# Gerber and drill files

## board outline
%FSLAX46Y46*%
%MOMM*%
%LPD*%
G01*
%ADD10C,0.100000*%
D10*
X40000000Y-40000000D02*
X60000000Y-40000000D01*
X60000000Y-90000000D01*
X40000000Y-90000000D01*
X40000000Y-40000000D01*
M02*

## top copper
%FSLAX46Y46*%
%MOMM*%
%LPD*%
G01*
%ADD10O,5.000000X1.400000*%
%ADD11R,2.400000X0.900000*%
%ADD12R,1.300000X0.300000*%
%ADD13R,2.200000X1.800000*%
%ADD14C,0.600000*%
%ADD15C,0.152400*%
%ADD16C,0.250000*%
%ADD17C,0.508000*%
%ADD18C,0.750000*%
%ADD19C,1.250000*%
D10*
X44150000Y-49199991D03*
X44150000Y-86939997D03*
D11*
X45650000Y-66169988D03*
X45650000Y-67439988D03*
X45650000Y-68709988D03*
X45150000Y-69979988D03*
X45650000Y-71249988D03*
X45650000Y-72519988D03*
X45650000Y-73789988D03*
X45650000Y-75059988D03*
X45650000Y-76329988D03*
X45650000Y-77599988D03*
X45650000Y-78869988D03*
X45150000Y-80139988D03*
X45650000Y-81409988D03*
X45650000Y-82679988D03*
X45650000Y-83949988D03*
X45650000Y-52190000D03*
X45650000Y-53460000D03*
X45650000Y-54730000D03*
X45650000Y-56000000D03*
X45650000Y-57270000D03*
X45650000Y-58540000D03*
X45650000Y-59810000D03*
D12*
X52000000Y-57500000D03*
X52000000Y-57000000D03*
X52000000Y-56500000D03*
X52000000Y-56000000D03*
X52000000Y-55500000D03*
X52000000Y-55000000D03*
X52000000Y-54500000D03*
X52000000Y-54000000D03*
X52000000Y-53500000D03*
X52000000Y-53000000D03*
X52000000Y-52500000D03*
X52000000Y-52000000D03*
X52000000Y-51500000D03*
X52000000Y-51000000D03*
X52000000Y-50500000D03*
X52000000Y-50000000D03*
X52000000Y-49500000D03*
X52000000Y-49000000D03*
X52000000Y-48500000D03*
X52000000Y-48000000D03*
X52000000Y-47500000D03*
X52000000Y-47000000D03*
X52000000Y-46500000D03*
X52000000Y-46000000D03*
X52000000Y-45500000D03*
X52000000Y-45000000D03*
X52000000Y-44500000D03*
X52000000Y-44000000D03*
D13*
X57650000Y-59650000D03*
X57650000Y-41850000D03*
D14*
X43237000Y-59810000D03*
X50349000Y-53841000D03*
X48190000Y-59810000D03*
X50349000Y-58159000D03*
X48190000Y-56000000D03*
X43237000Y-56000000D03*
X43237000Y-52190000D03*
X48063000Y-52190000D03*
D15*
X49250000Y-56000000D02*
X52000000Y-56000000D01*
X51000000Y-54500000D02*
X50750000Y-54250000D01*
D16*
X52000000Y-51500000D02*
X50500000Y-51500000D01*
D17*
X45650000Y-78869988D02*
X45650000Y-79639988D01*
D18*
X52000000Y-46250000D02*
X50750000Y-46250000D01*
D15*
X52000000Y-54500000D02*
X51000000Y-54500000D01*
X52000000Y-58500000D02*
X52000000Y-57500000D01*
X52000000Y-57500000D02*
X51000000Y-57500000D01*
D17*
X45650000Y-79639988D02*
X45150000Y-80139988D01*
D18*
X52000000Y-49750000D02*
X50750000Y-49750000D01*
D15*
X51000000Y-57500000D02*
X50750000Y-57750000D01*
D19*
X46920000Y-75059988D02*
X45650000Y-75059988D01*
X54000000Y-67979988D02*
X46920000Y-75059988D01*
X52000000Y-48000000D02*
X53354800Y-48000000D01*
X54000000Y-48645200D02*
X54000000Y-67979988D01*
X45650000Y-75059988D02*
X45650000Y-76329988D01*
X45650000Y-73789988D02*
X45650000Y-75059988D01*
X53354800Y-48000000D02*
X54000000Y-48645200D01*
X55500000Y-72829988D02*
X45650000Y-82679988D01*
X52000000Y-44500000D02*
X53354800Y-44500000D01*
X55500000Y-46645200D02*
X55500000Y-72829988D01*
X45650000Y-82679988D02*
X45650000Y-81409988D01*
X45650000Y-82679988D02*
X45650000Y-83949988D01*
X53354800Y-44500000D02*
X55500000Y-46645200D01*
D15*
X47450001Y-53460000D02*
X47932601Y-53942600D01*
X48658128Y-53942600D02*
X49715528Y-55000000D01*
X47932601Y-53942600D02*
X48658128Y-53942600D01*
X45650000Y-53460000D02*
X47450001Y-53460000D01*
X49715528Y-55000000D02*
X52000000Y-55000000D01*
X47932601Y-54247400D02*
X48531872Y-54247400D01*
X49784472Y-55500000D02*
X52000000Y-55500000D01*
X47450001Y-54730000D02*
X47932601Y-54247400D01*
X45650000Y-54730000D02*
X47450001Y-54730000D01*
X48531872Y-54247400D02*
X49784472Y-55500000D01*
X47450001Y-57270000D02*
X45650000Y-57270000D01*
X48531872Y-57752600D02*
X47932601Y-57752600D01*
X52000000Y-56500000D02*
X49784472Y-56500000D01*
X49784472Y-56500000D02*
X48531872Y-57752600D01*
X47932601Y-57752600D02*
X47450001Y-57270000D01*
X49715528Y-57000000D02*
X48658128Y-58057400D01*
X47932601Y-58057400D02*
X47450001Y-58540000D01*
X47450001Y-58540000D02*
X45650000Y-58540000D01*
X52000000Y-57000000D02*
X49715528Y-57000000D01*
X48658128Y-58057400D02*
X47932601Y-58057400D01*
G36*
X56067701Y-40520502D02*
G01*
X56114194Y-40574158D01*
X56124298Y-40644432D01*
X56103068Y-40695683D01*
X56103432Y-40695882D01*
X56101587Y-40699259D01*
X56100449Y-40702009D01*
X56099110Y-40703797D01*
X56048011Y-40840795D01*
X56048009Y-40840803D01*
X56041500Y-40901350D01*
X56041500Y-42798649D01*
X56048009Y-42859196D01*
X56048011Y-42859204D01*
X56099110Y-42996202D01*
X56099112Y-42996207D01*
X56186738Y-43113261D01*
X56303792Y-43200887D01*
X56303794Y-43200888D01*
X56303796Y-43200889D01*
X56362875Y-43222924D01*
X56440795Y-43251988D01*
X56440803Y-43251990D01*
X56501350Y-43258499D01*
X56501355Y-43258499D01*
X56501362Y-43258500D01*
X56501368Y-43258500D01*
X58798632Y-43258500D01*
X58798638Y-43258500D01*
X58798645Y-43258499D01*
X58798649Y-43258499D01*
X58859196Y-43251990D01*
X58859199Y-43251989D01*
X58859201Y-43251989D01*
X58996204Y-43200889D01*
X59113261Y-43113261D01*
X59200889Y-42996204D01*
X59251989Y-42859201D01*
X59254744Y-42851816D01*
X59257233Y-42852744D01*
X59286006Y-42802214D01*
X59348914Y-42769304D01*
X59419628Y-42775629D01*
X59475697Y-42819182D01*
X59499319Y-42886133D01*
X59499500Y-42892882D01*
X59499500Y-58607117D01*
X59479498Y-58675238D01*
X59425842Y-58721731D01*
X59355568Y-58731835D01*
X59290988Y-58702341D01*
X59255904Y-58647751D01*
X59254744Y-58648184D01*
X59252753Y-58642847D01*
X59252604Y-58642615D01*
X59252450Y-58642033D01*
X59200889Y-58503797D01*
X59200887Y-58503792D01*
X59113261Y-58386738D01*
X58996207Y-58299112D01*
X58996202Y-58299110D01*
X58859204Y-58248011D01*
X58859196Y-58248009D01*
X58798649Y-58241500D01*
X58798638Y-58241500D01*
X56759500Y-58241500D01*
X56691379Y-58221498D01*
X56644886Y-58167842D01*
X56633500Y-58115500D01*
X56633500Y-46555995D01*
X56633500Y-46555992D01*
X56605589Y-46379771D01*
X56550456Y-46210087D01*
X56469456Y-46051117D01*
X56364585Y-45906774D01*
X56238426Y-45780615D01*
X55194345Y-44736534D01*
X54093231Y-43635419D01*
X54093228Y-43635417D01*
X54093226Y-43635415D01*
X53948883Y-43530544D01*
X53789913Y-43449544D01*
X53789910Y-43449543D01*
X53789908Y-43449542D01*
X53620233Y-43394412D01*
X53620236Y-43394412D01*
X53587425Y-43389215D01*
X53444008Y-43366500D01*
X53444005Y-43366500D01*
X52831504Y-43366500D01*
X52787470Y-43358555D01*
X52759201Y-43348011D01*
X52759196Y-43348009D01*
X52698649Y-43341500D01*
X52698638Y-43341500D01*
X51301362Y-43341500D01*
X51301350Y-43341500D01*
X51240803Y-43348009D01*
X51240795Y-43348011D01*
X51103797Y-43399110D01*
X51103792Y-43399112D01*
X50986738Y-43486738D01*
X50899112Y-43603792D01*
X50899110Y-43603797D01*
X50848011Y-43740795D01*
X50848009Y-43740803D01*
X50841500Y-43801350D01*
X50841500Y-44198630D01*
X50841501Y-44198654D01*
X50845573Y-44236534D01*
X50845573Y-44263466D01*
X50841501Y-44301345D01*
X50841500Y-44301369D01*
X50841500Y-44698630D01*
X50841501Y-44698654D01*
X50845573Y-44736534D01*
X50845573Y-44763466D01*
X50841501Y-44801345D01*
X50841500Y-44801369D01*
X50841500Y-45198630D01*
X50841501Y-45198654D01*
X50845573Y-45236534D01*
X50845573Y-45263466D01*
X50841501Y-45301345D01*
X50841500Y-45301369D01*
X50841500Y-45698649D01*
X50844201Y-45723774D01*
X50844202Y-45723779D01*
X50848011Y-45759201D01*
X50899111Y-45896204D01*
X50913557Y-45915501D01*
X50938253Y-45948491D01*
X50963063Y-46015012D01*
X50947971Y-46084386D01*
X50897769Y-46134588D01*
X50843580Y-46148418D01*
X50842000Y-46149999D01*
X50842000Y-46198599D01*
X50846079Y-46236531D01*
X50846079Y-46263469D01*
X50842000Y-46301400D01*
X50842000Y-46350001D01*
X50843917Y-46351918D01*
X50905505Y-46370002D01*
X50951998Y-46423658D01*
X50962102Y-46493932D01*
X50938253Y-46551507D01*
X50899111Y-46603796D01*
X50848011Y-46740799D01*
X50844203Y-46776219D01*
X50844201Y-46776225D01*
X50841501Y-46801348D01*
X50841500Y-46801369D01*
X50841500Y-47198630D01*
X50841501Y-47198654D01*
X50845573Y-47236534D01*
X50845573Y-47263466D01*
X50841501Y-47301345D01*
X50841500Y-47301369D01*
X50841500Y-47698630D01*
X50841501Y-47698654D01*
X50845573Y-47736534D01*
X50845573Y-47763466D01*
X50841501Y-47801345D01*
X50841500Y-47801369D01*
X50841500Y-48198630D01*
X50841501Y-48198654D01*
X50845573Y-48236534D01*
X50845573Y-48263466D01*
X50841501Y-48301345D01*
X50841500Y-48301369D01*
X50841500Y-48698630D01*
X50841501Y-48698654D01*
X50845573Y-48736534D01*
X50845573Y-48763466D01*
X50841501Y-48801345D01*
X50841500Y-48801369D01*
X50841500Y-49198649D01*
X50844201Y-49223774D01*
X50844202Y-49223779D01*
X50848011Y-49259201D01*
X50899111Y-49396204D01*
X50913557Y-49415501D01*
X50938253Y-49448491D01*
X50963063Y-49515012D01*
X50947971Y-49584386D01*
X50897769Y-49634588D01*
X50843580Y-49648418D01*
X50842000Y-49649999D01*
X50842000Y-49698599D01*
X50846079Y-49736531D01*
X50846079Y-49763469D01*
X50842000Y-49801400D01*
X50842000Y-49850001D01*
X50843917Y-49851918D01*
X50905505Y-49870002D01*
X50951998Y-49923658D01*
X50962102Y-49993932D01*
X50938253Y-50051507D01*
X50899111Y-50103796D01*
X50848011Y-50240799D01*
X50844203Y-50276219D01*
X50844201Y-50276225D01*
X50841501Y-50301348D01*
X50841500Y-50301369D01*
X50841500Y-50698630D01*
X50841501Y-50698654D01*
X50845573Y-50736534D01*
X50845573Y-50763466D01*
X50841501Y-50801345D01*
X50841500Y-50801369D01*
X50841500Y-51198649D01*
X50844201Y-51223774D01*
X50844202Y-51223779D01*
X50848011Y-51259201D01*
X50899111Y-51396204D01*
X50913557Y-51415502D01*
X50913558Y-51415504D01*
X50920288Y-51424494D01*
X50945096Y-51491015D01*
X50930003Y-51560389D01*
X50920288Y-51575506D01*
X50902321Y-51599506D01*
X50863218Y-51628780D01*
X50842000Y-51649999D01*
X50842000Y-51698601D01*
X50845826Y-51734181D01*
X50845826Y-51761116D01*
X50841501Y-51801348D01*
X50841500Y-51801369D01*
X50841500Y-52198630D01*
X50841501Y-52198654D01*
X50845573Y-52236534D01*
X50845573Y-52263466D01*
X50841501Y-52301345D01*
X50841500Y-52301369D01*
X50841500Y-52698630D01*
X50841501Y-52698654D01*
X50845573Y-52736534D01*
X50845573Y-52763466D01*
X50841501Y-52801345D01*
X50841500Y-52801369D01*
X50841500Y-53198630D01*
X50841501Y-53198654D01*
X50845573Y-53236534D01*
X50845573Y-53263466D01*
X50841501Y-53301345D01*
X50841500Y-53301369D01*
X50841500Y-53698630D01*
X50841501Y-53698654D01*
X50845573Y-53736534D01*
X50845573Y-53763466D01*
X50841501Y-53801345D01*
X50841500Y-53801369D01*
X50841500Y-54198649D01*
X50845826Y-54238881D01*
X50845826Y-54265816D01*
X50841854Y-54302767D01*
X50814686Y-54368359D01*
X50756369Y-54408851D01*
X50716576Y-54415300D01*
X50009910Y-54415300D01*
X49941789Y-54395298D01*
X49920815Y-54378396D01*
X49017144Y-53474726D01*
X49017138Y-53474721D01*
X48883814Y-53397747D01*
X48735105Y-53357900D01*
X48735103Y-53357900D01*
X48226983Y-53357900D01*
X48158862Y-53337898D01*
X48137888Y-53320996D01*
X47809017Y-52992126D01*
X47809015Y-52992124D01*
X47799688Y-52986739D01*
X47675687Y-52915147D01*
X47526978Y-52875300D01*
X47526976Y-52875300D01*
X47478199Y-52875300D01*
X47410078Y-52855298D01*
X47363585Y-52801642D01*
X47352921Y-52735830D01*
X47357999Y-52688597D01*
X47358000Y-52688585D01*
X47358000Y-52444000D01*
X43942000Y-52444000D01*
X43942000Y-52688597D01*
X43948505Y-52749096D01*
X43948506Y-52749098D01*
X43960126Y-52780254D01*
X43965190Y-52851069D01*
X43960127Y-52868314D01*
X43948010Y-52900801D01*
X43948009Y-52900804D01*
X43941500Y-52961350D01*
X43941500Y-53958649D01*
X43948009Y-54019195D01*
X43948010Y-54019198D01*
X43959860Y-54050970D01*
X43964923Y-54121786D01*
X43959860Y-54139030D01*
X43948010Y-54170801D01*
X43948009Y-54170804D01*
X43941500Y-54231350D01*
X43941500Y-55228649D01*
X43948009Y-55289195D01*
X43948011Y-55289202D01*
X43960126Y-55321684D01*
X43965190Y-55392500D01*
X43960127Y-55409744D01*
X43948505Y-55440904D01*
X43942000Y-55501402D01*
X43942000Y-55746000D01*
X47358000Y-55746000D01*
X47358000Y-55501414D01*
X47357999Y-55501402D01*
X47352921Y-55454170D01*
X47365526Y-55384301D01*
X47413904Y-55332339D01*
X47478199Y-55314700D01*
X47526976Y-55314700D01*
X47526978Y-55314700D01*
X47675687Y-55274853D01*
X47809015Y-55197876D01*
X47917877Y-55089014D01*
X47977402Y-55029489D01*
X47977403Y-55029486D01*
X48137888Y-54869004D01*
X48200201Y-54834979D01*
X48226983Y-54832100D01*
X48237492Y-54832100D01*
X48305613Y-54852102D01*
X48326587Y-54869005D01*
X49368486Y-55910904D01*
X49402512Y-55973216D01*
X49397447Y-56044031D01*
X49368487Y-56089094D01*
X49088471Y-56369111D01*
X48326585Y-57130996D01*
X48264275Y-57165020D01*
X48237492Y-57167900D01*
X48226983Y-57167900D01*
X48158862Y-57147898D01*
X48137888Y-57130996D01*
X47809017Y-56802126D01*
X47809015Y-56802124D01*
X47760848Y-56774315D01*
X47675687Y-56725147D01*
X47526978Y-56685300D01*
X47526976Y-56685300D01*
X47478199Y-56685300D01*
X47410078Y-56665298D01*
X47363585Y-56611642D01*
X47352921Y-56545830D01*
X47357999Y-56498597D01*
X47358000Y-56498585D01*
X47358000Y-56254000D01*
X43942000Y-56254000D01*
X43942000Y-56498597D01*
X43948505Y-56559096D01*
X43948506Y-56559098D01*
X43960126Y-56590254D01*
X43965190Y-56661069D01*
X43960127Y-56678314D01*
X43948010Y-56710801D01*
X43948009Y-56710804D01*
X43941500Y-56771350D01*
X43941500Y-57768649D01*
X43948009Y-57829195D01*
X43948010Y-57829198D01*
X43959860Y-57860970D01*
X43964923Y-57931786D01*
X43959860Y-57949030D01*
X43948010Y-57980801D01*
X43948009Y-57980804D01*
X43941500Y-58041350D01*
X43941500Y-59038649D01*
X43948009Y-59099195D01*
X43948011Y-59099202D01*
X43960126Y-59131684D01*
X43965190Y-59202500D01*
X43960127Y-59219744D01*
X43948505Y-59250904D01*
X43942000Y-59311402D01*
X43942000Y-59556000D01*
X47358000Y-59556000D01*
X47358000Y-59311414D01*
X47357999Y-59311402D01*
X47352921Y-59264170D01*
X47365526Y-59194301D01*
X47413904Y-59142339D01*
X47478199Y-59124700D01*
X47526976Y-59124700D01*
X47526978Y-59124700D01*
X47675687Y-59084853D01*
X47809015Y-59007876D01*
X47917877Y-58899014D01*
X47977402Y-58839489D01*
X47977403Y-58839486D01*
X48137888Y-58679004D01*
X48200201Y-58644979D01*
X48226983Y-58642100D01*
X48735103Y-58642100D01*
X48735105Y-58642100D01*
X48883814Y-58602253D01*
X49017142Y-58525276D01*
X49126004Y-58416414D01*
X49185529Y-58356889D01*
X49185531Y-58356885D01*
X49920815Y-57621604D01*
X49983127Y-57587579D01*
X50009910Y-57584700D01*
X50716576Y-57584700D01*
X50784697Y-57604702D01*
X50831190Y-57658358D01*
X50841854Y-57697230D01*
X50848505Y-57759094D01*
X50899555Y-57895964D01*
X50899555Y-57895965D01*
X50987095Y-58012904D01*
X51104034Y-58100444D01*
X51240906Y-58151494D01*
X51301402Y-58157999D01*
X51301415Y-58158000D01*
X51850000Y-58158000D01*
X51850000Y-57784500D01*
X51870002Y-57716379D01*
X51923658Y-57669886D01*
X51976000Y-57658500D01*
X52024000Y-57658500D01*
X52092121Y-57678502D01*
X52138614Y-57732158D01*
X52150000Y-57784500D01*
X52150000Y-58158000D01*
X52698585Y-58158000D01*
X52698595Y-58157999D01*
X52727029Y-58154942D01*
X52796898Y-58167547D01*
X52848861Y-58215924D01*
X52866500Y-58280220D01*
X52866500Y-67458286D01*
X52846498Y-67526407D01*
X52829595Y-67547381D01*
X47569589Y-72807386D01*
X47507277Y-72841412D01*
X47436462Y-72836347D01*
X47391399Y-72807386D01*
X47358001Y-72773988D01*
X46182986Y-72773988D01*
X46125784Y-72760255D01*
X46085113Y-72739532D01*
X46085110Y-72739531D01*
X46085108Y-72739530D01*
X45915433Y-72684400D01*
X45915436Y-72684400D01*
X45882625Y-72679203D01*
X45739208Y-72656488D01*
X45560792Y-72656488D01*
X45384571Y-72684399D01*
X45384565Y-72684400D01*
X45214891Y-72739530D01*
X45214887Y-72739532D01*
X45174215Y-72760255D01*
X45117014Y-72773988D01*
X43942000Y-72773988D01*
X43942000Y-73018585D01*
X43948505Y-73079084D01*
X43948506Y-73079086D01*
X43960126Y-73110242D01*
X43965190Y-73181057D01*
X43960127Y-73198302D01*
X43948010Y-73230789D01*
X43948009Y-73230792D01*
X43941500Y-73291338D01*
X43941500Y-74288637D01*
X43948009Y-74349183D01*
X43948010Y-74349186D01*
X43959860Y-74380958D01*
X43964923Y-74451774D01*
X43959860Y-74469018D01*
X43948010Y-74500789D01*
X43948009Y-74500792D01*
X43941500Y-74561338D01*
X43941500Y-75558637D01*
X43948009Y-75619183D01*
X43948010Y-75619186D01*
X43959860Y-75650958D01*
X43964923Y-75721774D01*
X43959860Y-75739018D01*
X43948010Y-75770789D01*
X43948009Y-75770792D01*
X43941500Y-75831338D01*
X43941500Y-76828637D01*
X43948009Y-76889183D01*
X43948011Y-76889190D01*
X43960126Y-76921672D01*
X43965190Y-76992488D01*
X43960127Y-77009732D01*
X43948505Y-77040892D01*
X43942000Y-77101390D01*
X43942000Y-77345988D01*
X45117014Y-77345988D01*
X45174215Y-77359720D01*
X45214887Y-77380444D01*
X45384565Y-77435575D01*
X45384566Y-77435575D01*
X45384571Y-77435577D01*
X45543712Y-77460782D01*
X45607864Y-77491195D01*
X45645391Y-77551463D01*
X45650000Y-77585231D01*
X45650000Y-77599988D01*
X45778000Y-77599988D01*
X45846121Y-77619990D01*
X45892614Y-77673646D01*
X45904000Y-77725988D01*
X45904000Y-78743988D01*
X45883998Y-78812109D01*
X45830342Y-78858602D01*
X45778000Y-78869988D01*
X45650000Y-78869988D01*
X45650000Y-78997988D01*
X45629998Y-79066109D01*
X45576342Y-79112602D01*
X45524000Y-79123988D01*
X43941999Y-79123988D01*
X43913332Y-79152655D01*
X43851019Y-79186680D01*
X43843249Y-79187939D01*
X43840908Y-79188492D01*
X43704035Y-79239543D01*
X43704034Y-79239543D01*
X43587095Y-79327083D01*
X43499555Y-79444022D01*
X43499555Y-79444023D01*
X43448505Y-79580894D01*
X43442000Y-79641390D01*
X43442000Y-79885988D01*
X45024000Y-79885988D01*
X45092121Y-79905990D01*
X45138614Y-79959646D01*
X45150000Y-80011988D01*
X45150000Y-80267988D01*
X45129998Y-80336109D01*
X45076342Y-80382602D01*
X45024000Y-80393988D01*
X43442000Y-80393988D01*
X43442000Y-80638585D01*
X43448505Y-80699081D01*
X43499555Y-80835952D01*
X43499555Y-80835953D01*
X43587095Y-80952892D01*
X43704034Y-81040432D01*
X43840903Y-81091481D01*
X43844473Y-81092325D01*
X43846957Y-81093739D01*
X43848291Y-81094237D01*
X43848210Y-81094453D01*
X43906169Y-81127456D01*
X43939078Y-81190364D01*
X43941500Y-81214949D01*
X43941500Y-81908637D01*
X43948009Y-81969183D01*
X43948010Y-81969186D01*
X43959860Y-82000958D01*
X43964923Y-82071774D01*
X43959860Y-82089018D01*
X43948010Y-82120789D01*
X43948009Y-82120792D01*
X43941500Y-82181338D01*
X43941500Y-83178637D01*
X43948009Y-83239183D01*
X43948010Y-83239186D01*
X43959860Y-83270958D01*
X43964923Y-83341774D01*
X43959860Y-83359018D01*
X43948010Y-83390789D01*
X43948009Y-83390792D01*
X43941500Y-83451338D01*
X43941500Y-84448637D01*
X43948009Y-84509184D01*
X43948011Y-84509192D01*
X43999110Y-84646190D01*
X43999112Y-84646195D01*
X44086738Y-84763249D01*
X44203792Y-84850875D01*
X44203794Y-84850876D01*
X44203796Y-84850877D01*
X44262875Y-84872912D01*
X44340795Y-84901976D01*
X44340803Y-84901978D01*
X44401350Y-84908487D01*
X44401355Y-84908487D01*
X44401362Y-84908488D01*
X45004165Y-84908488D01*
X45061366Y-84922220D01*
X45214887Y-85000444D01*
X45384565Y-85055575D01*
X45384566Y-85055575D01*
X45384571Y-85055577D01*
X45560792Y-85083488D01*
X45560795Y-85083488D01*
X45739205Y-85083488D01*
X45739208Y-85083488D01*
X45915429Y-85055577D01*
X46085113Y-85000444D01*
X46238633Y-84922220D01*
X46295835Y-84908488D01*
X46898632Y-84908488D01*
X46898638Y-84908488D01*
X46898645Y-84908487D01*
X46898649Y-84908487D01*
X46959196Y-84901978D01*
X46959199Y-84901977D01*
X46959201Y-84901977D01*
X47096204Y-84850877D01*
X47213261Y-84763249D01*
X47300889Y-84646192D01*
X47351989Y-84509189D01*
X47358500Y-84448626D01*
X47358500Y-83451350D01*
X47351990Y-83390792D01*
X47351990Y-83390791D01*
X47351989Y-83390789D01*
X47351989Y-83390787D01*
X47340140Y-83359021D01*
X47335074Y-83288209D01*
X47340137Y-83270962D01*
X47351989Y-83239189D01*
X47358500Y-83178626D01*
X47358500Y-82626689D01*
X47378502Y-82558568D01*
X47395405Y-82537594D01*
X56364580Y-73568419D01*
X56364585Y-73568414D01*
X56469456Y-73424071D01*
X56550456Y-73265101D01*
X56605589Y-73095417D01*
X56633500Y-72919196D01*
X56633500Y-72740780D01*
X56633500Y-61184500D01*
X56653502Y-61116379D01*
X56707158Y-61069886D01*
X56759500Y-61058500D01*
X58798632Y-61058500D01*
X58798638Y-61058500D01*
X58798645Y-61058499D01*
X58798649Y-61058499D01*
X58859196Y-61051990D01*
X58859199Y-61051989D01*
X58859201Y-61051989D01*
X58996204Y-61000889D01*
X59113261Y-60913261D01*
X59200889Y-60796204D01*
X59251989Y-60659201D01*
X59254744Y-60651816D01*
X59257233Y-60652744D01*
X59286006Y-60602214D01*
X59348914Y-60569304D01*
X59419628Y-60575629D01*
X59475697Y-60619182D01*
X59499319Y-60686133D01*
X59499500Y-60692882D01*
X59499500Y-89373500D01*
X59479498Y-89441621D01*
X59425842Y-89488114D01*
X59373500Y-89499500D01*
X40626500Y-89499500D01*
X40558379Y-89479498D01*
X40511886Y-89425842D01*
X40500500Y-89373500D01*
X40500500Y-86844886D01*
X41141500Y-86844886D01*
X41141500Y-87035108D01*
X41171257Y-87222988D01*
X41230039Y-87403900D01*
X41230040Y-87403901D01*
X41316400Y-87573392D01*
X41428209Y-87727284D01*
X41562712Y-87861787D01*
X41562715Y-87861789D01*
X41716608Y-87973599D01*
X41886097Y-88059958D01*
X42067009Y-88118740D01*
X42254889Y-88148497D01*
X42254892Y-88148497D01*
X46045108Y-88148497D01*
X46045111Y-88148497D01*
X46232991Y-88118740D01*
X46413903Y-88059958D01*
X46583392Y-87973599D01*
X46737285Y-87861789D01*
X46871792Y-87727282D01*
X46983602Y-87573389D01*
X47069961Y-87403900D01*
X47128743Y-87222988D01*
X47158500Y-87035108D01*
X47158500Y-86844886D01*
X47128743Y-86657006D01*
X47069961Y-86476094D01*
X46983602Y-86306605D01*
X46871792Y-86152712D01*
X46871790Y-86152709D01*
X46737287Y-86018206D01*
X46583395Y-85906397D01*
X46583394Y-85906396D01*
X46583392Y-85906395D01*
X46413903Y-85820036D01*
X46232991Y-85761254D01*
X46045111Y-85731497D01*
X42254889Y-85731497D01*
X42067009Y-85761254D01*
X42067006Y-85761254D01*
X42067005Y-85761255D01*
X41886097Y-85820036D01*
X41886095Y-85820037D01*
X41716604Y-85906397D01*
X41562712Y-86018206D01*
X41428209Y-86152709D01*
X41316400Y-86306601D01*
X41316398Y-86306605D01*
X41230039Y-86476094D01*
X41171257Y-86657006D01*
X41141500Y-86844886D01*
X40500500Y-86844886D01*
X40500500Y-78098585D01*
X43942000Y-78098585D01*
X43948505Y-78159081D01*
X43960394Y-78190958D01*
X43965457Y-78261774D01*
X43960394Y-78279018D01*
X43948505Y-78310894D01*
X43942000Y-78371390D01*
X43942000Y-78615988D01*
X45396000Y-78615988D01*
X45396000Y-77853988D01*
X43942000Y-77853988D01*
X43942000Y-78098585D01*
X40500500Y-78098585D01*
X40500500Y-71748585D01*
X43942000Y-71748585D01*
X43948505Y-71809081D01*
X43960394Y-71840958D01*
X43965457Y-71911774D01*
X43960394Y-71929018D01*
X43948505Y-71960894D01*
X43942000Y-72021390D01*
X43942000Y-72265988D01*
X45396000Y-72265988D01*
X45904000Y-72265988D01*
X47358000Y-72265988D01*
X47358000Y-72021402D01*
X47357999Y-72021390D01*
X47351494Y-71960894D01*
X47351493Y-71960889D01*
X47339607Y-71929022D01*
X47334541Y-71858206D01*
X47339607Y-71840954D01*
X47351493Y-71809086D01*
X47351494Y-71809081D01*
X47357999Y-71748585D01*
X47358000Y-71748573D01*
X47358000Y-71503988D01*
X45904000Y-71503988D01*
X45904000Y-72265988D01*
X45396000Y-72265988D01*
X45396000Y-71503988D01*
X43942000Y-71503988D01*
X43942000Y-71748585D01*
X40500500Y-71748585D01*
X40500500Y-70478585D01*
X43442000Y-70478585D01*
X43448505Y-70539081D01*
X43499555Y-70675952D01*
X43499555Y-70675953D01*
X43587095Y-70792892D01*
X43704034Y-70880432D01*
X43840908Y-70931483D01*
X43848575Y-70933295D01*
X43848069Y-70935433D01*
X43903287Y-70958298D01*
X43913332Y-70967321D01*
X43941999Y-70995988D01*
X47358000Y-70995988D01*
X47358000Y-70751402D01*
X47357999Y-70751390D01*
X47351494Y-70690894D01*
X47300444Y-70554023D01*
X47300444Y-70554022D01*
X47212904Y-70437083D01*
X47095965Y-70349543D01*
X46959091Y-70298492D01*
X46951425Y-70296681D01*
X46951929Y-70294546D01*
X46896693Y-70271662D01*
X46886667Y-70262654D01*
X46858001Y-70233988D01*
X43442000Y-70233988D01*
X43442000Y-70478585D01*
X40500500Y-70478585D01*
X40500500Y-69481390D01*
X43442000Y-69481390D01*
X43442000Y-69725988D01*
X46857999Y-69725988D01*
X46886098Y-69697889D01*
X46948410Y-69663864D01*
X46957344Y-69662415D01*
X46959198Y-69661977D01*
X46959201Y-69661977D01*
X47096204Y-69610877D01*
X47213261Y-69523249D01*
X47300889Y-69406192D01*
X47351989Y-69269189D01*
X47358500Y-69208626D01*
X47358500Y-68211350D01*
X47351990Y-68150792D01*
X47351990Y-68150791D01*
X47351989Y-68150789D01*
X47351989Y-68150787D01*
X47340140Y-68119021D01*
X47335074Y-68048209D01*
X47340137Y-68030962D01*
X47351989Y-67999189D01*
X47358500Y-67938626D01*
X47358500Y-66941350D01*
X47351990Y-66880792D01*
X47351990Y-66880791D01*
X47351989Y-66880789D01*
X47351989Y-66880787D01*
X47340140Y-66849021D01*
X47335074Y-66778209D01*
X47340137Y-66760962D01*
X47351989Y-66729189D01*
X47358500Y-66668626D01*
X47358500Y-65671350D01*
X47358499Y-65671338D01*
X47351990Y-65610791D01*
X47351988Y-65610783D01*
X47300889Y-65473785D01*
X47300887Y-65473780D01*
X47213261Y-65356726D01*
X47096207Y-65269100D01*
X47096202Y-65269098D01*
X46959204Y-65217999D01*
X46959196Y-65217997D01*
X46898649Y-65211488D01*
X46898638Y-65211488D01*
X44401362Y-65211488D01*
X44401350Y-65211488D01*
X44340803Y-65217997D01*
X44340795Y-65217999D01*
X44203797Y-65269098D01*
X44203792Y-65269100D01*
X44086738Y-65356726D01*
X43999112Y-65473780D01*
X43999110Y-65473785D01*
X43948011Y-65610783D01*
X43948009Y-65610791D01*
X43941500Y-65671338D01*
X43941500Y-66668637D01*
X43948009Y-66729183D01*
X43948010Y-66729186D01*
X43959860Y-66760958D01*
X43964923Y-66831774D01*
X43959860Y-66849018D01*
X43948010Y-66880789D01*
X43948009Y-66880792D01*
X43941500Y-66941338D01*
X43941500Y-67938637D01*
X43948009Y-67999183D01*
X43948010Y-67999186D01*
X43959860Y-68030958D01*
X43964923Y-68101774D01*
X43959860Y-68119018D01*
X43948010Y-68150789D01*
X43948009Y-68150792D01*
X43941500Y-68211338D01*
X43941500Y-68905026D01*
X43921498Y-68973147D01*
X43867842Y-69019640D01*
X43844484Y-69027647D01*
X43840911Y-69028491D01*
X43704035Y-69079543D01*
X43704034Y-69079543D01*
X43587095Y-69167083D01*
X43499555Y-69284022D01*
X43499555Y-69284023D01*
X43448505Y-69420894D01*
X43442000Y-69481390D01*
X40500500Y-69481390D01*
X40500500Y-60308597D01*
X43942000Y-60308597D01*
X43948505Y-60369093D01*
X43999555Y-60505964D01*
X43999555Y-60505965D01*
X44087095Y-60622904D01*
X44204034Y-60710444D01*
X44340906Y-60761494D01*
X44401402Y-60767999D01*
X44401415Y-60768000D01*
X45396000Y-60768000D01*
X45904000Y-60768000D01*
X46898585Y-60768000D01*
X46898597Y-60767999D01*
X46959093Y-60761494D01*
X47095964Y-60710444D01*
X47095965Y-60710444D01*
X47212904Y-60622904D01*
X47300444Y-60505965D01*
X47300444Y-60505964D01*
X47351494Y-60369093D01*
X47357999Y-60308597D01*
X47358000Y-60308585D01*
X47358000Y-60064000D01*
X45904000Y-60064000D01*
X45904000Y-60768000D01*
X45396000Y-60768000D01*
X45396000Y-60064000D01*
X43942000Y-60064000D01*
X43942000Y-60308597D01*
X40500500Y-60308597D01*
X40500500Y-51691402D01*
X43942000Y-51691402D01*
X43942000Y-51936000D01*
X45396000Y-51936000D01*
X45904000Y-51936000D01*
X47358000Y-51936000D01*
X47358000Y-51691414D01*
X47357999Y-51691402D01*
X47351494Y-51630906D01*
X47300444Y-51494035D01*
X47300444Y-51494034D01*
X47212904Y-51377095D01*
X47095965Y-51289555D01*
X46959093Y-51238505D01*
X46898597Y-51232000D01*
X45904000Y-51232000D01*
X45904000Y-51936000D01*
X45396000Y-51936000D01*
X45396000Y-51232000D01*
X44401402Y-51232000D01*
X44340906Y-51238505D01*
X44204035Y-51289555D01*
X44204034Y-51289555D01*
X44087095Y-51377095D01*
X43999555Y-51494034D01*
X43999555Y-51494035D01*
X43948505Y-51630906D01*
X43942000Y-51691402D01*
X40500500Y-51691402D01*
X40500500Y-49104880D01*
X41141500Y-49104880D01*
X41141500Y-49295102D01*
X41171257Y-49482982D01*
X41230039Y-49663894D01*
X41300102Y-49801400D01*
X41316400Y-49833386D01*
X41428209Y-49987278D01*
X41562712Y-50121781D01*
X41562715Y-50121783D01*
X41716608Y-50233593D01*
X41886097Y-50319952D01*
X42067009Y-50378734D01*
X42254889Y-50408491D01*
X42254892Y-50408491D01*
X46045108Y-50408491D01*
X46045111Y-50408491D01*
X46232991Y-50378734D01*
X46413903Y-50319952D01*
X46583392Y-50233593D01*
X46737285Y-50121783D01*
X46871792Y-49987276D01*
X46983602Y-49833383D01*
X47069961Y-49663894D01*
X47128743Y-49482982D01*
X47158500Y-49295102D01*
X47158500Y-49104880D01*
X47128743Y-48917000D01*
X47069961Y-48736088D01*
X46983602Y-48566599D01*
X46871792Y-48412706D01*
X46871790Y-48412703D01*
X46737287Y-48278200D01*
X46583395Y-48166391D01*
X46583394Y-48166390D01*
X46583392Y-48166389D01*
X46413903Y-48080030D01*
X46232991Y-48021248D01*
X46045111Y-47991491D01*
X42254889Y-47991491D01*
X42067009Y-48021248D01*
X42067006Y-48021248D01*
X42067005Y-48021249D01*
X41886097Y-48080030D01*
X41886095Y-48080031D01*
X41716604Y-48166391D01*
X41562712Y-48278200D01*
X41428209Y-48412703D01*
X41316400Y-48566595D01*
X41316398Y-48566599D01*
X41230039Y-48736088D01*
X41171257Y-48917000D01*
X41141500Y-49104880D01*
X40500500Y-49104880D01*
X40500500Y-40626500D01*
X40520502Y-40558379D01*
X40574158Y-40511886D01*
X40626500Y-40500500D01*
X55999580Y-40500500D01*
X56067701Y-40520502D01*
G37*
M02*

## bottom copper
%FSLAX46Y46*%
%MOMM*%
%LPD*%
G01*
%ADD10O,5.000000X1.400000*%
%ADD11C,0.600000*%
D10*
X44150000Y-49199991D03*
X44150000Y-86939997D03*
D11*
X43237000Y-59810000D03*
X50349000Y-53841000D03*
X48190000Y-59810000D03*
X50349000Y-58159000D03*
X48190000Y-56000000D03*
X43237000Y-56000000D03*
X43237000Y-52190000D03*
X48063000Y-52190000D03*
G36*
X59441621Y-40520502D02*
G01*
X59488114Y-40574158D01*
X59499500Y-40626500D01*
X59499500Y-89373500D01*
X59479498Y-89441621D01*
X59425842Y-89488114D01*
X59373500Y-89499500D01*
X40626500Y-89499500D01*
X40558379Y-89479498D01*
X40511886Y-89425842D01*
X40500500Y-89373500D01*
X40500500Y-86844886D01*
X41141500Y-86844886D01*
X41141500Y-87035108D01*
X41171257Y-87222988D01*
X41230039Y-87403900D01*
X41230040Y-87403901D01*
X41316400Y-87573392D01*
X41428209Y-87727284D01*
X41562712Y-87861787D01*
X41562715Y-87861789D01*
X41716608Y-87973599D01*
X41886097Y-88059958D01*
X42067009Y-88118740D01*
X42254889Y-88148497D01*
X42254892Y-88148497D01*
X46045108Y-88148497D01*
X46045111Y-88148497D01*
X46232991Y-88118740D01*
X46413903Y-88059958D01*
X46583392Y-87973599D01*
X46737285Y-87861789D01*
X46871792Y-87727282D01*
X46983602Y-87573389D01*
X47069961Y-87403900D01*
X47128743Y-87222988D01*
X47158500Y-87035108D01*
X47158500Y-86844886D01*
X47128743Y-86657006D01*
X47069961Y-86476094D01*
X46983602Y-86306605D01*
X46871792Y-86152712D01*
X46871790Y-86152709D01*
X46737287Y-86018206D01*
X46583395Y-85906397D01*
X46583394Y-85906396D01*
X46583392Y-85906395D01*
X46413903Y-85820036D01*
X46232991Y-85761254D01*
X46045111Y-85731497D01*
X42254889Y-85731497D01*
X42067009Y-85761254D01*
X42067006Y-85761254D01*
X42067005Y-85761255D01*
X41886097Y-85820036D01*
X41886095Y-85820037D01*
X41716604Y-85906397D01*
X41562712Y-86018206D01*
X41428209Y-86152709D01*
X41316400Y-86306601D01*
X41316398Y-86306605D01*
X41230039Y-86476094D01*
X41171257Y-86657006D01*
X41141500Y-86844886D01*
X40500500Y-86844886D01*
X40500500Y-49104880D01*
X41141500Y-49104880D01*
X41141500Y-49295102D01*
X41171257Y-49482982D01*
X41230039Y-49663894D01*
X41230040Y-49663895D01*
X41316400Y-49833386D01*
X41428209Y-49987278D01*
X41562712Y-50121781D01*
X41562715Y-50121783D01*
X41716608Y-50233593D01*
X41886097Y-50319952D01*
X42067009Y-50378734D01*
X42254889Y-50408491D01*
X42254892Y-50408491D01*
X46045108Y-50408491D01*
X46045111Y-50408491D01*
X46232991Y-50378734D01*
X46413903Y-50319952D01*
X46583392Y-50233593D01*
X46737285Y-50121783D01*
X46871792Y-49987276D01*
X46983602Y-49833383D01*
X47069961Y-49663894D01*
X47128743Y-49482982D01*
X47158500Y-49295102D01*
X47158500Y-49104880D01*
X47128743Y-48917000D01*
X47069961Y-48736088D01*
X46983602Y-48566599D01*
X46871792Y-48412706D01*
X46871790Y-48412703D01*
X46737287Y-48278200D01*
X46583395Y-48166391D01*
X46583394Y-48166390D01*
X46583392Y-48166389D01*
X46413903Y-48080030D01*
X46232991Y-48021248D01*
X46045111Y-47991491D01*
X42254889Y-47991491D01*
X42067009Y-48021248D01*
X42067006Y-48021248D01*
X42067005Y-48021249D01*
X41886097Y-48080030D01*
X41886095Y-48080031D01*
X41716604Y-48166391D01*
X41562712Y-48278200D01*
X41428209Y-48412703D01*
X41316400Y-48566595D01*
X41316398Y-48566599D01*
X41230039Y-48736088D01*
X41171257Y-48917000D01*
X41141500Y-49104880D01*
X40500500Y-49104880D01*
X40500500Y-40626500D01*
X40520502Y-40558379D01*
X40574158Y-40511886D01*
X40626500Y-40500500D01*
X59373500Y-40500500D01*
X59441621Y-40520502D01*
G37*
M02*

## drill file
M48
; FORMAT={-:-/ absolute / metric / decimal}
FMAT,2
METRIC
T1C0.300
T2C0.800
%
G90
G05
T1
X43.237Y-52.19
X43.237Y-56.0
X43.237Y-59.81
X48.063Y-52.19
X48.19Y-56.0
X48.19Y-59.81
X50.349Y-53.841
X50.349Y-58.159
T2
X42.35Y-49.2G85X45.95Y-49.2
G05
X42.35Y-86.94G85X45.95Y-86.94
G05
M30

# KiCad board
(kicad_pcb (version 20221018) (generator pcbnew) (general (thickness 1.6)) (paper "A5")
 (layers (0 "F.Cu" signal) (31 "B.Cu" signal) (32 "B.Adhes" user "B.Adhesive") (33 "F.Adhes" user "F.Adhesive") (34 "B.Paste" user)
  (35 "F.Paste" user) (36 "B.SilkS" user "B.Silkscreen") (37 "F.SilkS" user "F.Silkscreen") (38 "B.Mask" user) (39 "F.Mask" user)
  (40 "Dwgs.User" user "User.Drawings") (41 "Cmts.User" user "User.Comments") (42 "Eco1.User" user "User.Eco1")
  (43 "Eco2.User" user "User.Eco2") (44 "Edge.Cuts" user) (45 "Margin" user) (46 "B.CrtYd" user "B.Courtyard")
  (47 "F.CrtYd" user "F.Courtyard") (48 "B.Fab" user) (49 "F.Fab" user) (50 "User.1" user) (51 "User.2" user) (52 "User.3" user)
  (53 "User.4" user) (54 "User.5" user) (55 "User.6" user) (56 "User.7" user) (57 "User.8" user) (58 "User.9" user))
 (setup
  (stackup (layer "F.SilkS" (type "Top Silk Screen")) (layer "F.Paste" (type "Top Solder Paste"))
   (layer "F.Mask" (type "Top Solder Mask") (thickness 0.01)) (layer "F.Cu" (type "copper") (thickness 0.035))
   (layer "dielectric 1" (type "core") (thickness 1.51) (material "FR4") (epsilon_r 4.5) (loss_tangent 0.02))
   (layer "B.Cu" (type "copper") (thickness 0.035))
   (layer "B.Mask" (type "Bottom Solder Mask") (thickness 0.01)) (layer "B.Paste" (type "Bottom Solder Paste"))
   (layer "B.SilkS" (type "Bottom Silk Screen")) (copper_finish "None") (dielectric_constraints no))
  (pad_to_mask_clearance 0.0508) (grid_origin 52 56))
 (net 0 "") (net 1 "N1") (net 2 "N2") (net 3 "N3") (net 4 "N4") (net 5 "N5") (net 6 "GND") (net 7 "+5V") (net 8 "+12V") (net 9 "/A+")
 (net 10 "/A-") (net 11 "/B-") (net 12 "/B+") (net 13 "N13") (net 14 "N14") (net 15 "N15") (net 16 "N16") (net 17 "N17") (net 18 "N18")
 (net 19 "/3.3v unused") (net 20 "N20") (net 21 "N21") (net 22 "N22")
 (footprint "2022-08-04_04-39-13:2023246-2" (layer "F.Cu") (at 45.6246 52.245794 -90)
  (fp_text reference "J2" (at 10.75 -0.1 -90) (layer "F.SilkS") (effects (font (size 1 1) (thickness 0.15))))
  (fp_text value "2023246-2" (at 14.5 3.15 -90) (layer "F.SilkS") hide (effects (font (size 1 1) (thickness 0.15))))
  (pad "23" thru_hole oval (at -3.045803 1.4746) (size 5 1.4) (drill oval 4.4 0.8) (layers "*.Cu" "*.Mask") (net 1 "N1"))
  (pad "24" thru_hole oval (at 34.694203 1.4746) (size 5 1.4) (drill oval 4.4 0.8) (layers "*.Cu" "*.Mask") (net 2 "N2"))
  (pad "P1" smd rect (at 13.924194 -0.0254 270) (size 0.9 2.4) (layers "F.Cu" "F.Paste" "F.Mask") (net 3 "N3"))
  (pad "P2" smd rect (at 15.194194 -0.0254 270) (size 0.9 2.4) (layers "F.Cu" "F.Paste" "F.Mask") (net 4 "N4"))
  (pad "P3" smd rect (at 16.464194 -0.0254 270) (size 0.9 2.4) (layers "F.Cu" "F.Paste" "F.Mask") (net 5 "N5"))
  (pad "P4" smd rect (at 17.734194 0.4746 270) (size 0.9 2.4) (layers "F.Cu" "F.Paste" "F.Mask") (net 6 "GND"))
  (pad "P5" smd rect (at 19.004194 -0.0254 270) (size 0.9 2.4) (layers "F.Cu" "F.Paste" "F.Mask") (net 6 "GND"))
  (pad "P6" smd rect (at 20.274194 -0.0254 270) (size 0.9 2.4) (layers "F.Cu" "F.Paste" "F.Mask") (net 6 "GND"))
  (pad "P7" smd rect (at 21.544194 -0.0254 270) (size 0.9 2.4) (layers "F.Cu" "F.Paste" "F.Mask") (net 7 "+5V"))
  (pad "P8" smd rect (at 22.814194 -0.0254 270) (size 0.9 2.4) (layers "F.Cu" "F.Paste" "F.Mask") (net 7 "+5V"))
  (pad "P9" smd rect (at 24.084194 -0.0254 270) (size 0.9 2.4) (layers "F.Cu" "F.Paste" "F.Mask") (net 7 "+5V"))
  (pad "P10" smd rect (at 25.354194 -0.0254 270) (size 0.9 2.4) (layers "F.Cu" "F.Paste" "F.Mask") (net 6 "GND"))
  (pad "P11" smd rect (at 26.624194 -0.0254 270) (size 0.9 2.4) (layers "F.Cu" "F.Paste" "F.Mask") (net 6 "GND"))
  (pad "P12" smd rect (at 27.894194 0.4746 270) (size 0.9 2.4) (layers "F.Cu" "F.Paste" "F.Mask") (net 6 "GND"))
  (pad "P13" smd rect (at 29.164194 -0.0254 270) (size 0.9 2.4) (layers "F.Cu" "F.Paste" "F.Mask") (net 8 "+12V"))
  (pad "P14" smd rect (at 30.434194 -0.0254 270) (size 0.9 2.4) (layers "F.Cu" "F.Paste" "F.Mask") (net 8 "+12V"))
  (pad "P15" smd rect (at 31.704194 -0.0254 270) (size 0.9 2.4) (layers "F.Cu" "F.Paste" "F.Mask") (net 8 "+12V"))
  (pad "S1" smd rect (at -0.055794 -0.0254 270) (size 0.9 2.4) (layers "F.Cu" "F.Paste" "F.Mask") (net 6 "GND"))
  (pad "S2" smd rect (at 1.214206 -0.0254 270) (size 0.9 2.4) (layers "F.Cu" "F.Paste" "F.Mask") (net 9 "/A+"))
  (pad "S3" smd rect (at 2.484206 -0.0254 270) (size 0.9 2.4) (layers "F.Cu" "F.Paste" "F.Mask") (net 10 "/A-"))
  (pad "S4" smd rect (at 3.754206 -0.0254 270) (size 0.9 2.4) (layers "F.Cu" "F.Paste" "F.Mask") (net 6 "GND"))
  (pad "S5" smd rect (at 5.024206 -0.0254 270) (size 0.9 2.4) (layers "F.Cu" "F.Paste" "F.Mask") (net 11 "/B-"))
  (pad "S6" smd rect (at 6.294206 -0.0254 270) (size 0.9 2.4) (layers "F.Cu" "F.Paste" "F.Mask") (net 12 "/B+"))
  (pad "S7" smd rect (at 7.564206 -0.0254 270) (size 0.9 2.4) (layers "F.Cu" "F.Paste" "F.Mask") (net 6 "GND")))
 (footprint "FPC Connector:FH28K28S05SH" (layer "F.Cu") (at 55.575 50.75 90)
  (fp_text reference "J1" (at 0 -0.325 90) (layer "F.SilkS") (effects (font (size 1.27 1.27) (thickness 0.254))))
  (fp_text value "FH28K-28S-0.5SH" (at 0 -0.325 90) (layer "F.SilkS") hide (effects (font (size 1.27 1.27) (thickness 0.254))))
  (pad "1" smd rect (at -6.75 -3.575 90) (size 0.3 1.3) (layers "F.Cu" "F.Paste" "F.Mask") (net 6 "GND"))
  (pad "2" smd rect (at -6.25 -3.575 90) (size 0.3 1.3) (layers "F.Cu" "F.Paste" "F.Mask") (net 12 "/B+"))
  (pad "3" smd rect (at -5.75 -3.575 90) (size 0.3 1.3) (layers "F.Cu" "F.Paste" "F.Mask") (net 11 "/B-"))
  (pad "4" smd rect (at -5.25 -3.575 90) (size 0.3 1.3) (layers "F.Cu" "F.Paste" "F.Mask") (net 6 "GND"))
  (pad "5" smd rect (at -4.75 -3.575 90) (size 0.3 1.3) (layers "F.Cu" "F.Paste" "F.Mask") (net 10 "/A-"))
  (pad "6" smd rect (at -4.25 -3.575 90) (size 0.3 1.3) (layers "F.Cu" "F.Paste" "F.Mask") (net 9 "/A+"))
  (pad "7" smd rect (at -3.75 -3.575 90) (size 0.3 1.3) (layers "F.Cu" "F.Paste" "F.Mask") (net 6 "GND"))
  (pad "8" smd rect (at -3.25 -3.575 90) (size 0.3 1.3) (layers "F.Cu" "F.Paste" "F.Mask") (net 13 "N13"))
  (pad "9" smd rect (at -2.75 -3.575 90) (size 0.3 1.3) (layers "F.Cu" "F.Paste" "F.Mask") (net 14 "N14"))
  (pad "10" smd rect (at -2.25 -3.575 90) (size 0.3 1.3) (layers "F.Cu" "F.Paste" "F.Mask") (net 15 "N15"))
  (pad "11" smd rect (at -1.75 -3.575 90) (size 0.3 1.3) (layers "F.Cu" "F.Paste" "F.Mask") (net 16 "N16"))
  (pad "12" smd rect (at -1.25 -3.575 90) (size 0.3 1.3) (layers "F.Cu" "F.Paste" "F.Mask") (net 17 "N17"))
  (pad "13" smd rect (at -0.75 -3.575 90) (size 0.3 1.3) (layers "F.Cu" "F.Paste" "F.Mask") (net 6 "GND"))
  (pad "14" smd rect (at -0.25 -3.575 90) (size 0.3 1.3) (layers "F.Cu" "F.Paste" "F.Mask") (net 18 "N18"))
  (pad "15" smd rect (at 0.25 -3.575 90) (size 0.3 1.3) (layers "F.Cu" "F.Paste" "F.Mask") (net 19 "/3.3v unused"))
  (pad "16" smd rect (at 0.75 -3.575 90) (size 0.3 1.3) (layers "F.Cu" "F.Paste" "F.Mask") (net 6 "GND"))
  (pad "17" smd rect (at 1.25 -3.575 90) (size 0.3 1.3) (layers "F.Cu" "F.Paste" "F.Mask") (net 6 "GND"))
  (pad "18" smd rect (at 1.75 -3.575 90) (size 0.3 1.3) (layers "F.Cu" "F.Paste" "F.Mask") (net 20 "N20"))
  (pad "19" smd rect (at 2.25 -3.575 90) (size 0.3 1.3) (layers "F.Cu" "F.Paste" "F.Mask") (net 7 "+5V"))
  (pad "20" smd rect (at 2.75 -3.575 90) (size 0.3 1.3) (layers "F.Cu" "F.Paste" "F.Mask") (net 7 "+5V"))
  (pad "21" smd rect (at 3.25 -3.575 90) (size 0.3 1.3) (layers "F.Cu" "F.Paste" "F.Mask") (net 7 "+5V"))
  (pad "22" smd rect (at 3.75 -3.575 90) (size 0.3 1.3) (layers "F.Cu" "F.Paste" "F.Mask") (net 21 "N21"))
  (pad "23" smd rect (at 4.25 -3.575 90) (size 0.3 1.3) (layers "F.Cu" "F.Paste" "F.Mask") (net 6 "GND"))
  (pad "24" smd rect (at 4.75 -3.575 90) (size 0.3 1.3) (layers "F.Cu" "F.Paste" "F.Mask") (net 6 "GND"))
  (pad "25" smd rect (at 5.25 -3.575 90) (size 0.3 1.3) (layers "F.Cu" "F.Paste" "F.Mask") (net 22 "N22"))
  (pad "26" smd rect (at 5.75 -3.575 90) (size 0.3 1.3) (layers "F.Cu" "F.Paste" "F.Mask") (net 8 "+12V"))
  (pad "27" smd rect (at 6.25 -3.575 90) (size 0.3 1.3) (layers "F.Cu" "F.Paste" "F.Mask") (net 8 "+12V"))
  (pad "28" smd rect (at 6.75 -3.575 90) (size 0.3 1.3) (layers "F.Cu" "F.Paste" "F.Mask") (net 8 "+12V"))
  (pad "MP1" smd rect (at -8.9 2.075 90) (size 1.8 2.2) (layers "F.Cu" "F.Paste" "F.Mask"))
  (pad "MP2" smd rect (at 8.9 2.075 90) (size 1.8 2.2) (layers "F.Cu" "F.Paste" "F.Mask")))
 (gr_rect (start 40 40) (end 60 90) (stroke (width 0.1) (type solid)) (fill none) (layer "Edge.Cuts"))
 (segment (start 49.25 56) (end 52 56) (width 0.1524) (layer "F.Cu") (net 6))
 (segment (start 51 54.5) (end 50.75 54.25) (width 0.1524) (layer "F.Cu") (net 6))
 (segment (start 52 51.5) (end 50.5 51.5) (width 0.25) (layer "F.Cu") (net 6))
 (segment (start 45.65 78.869988) (end 45.65 79.639988) (width 0.508) (layer "F.Cu") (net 6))
 (segment (start 52 46.25) (end 50.75 46.25) (width 0.75) (layer "F.Cu") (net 6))
 (segment (start 52 54.5) (end 51 54.5) (width 0.1524) (layer "F.Cu") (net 6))
 (segment (start 52 58.5) (end 52 57.5) (width 0.1524) (layer "F.Cu") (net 6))
 (segment (start 52 57.5) (end 51 57.5) (width 0.1524) (layer "F.Cu") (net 6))
 (segment (start 45.65 79.639988) (end 45.15 80.139988) (width 0.508) (layer "F.Cu") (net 6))
 (segment (start 52 49.75) (end 50.75 49.75) (width 0.75) (layer "F.Cu") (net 6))
 (segment (start 51 57.5) (end 50.75 57.75) (width 0.1524) (layer "F.Cu") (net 6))
 (via (at 43.237 59.81) (size 0.6) (drill 0.3) (layers "F.Cu" "B.Cu") (free) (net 6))
 (via (at 50.349 53.841) (size 0.6) (drill 0.3) (layers "F.Cu" "B.Cu") (free) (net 6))
 (via (at 48.19 59.81) (size 0.6) (drill 0.3) (layers "F.Cu" "B.Cu") (free) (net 6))
 (via (at 50.349 58.159) (size 0.6) (drill 0.3) (layers "F.Cu" "B.Cu") (free) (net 6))
 (via (at 48.19 56) (size 0.6) (drill 0.3) (layers "F.Cu" "B.Cu") (free) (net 6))
 (via (at 43.237 56) (size 0.6) (drill 0.3) (layers "F.Cu" "B.Cu") (free) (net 6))
 (via (at 43.237 52.19) (size 0.6) (drill 0.3) (layers "F.Cu" "B.Cu") (free) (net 6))
 (via (at 48.063 52.19) (size 0.6) (drill 0.3) (layers "F.Cu" "B.Cu") (free) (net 6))
 (segment (start 46.92 75.059988) (end 45.65 75.059988) (width 1.25) (layer "F.Cu") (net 7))
 (segment (start 54 67.979988) (end 46.92 75.059988) (width 1.25) (layer "F.Cu") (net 7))
 (segment (start 52 48) (end 53.3548 48) (width 1.25) (layer "F.Cu") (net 7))
 (segment (start 54 48.6452) (end 54 67.979988) (width 1.25) (layer "F.Cu") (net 7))
 (segment (start 45.65 75.059988) (end 45.65 76.329988) (width 1.25) (layer "F.Cu") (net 7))
 (segment (start 45.65 73.789988) (end 45.65 75.059988) (width 1.25) (layer "F.Cu") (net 7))
 (segment (start 53.3548 48) (end 54 48.6452) (width 1.25) (layer "F.Cu") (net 7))
 (segment (start 55.5 72.829988) (end 45.65 82.679988) (width 1.25) (layer "F.Cu") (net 8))
 (segment (start 52 44.5) (end 53.3548 44.5) (width 1.25) (layer "F.Cu") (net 8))
 (segment (start 55.5 46.6452) (end 55.5 72.829988) (width 1.25) (layer "F.Cu") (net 8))
 (segment (start 45.65 82.679988) (end 45.65 81.409988) (width 1.25) (layer "F.Cu") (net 8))
 (segment (start 45.65 82.679988) (end 45.65 83.949988) (width 1.25) (layer "F.Cu") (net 8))
 (segment (start 53.3548 44.5) (end 55.5 46.6452) (width 1.25) (layer "F.Cu") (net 8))
 (segment (start 47.450001 53.46) (end 47.932601 53.9426) (width 0.1524) (layer "F.Cu") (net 9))
 (segment (start 48.658128 53.9426) (end 49.715528 55) (width 0.1524) (layer "F.Cu") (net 9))
 (segment (start 47.932601 53.9426) (end 48.658128 53.9426) (width 0.1524) (layer "F.Cu") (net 9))
 (segment (start 45.65 53.46) (end 47.450001 53.46) (width 0.1524) (layer "F.Cu") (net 9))
 (segment (start 49.715528 55) (end 52 55) (width 0.1524) (layer "F.Cu") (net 9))
 (segment (start 47.932601 54.2474) (end 48.531872 54.2474) (width 0.1524) (layer "F.Cu") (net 10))
 (segment (start 49.784472 55.5) (end 52 55.5) (width 0.1524) (layer "F.Cu") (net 10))
 (segment (start 47.450001 54.73) (end 47.932601 54.2474) (width 0.1524) (layer "F.Cu") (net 10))
 (segment (start 45.65 54.73) (end 47.450001 54.73) (width 0.1524) (layer "F.Cu") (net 10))
 (segment (start 48.531872 54.2474) (end 49.784472 55.5) (width 0.1524) (layer "F.Cu") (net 10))
 (segment (start 47.450001 57.27) (end 45.65 57.27) (width 0.1524) (layer "F.Cu") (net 11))
 (segment (start 48.531872 57.7526) (end 47.932601 57.7526) (width 0.1524) (layer "F.Cu") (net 11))
 (segment (start 52 56.5) (end 49.784472 56.5) (width 0.1524) (layer "F.Cu") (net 11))
 (segment (start 49.784472 56.5) (end 48.531872 57.7526) (width 0.1524) (layer "F.Cu") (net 11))
 (segment (start 47.932601 57.7526) (end 47.450001 57.27) (width 0.1524) (layer "F.Cu") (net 11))
 (segment (start 49.715528 57) (end 48.658128 58.0574) (width 0.1524) (layer "F.Cu") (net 12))
 (segment (start 47.932601 58.0574) (end 47.450001 58.54) (width 0.1524) (layer "F.Cu") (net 12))
 (segment (start 47.450001 58.54) (end 45.65 58.54) (width 0.1524) (layer "F.Cu") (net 12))
 (segment (start 52 57) (end 49.715528 57) (width 0.1524) (layer "F.Cu") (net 12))
 (segment (start 48.658128 58.0574) (end 47.932601 58.0574) (width 0.1524) (layer "F.Cu") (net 12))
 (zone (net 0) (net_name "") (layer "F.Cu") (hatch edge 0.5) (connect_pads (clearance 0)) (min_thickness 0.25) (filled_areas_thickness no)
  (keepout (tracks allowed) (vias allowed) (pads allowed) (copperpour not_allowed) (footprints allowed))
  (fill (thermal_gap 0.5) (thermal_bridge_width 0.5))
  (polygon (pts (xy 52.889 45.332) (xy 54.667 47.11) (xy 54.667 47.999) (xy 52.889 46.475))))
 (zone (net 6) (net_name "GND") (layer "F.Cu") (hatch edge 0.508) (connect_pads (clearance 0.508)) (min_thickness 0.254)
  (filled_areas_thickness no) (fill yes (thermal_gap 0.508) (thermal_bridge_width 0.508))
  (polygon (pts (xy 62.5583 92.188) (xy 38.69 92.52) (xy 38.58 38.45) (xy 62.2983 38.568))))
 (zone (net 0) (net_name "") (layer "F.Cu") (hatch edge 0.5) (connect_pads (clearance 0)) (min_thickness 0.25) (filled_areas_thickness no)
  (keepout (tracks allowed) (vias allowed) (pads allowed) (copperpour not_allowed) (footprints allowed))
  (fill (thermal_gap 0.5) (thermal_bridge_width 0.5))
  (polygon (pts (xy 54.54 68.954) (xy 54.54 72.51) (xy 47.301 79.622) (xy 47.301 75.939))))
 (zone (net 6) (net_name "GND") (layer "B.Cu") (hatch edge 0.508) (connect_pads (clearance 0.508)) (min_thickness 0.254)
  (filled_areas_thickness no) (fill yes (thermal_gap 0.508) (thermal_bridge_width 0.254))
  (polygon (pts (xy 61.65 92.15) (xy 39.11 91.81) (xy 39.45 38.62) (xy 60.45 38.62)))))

